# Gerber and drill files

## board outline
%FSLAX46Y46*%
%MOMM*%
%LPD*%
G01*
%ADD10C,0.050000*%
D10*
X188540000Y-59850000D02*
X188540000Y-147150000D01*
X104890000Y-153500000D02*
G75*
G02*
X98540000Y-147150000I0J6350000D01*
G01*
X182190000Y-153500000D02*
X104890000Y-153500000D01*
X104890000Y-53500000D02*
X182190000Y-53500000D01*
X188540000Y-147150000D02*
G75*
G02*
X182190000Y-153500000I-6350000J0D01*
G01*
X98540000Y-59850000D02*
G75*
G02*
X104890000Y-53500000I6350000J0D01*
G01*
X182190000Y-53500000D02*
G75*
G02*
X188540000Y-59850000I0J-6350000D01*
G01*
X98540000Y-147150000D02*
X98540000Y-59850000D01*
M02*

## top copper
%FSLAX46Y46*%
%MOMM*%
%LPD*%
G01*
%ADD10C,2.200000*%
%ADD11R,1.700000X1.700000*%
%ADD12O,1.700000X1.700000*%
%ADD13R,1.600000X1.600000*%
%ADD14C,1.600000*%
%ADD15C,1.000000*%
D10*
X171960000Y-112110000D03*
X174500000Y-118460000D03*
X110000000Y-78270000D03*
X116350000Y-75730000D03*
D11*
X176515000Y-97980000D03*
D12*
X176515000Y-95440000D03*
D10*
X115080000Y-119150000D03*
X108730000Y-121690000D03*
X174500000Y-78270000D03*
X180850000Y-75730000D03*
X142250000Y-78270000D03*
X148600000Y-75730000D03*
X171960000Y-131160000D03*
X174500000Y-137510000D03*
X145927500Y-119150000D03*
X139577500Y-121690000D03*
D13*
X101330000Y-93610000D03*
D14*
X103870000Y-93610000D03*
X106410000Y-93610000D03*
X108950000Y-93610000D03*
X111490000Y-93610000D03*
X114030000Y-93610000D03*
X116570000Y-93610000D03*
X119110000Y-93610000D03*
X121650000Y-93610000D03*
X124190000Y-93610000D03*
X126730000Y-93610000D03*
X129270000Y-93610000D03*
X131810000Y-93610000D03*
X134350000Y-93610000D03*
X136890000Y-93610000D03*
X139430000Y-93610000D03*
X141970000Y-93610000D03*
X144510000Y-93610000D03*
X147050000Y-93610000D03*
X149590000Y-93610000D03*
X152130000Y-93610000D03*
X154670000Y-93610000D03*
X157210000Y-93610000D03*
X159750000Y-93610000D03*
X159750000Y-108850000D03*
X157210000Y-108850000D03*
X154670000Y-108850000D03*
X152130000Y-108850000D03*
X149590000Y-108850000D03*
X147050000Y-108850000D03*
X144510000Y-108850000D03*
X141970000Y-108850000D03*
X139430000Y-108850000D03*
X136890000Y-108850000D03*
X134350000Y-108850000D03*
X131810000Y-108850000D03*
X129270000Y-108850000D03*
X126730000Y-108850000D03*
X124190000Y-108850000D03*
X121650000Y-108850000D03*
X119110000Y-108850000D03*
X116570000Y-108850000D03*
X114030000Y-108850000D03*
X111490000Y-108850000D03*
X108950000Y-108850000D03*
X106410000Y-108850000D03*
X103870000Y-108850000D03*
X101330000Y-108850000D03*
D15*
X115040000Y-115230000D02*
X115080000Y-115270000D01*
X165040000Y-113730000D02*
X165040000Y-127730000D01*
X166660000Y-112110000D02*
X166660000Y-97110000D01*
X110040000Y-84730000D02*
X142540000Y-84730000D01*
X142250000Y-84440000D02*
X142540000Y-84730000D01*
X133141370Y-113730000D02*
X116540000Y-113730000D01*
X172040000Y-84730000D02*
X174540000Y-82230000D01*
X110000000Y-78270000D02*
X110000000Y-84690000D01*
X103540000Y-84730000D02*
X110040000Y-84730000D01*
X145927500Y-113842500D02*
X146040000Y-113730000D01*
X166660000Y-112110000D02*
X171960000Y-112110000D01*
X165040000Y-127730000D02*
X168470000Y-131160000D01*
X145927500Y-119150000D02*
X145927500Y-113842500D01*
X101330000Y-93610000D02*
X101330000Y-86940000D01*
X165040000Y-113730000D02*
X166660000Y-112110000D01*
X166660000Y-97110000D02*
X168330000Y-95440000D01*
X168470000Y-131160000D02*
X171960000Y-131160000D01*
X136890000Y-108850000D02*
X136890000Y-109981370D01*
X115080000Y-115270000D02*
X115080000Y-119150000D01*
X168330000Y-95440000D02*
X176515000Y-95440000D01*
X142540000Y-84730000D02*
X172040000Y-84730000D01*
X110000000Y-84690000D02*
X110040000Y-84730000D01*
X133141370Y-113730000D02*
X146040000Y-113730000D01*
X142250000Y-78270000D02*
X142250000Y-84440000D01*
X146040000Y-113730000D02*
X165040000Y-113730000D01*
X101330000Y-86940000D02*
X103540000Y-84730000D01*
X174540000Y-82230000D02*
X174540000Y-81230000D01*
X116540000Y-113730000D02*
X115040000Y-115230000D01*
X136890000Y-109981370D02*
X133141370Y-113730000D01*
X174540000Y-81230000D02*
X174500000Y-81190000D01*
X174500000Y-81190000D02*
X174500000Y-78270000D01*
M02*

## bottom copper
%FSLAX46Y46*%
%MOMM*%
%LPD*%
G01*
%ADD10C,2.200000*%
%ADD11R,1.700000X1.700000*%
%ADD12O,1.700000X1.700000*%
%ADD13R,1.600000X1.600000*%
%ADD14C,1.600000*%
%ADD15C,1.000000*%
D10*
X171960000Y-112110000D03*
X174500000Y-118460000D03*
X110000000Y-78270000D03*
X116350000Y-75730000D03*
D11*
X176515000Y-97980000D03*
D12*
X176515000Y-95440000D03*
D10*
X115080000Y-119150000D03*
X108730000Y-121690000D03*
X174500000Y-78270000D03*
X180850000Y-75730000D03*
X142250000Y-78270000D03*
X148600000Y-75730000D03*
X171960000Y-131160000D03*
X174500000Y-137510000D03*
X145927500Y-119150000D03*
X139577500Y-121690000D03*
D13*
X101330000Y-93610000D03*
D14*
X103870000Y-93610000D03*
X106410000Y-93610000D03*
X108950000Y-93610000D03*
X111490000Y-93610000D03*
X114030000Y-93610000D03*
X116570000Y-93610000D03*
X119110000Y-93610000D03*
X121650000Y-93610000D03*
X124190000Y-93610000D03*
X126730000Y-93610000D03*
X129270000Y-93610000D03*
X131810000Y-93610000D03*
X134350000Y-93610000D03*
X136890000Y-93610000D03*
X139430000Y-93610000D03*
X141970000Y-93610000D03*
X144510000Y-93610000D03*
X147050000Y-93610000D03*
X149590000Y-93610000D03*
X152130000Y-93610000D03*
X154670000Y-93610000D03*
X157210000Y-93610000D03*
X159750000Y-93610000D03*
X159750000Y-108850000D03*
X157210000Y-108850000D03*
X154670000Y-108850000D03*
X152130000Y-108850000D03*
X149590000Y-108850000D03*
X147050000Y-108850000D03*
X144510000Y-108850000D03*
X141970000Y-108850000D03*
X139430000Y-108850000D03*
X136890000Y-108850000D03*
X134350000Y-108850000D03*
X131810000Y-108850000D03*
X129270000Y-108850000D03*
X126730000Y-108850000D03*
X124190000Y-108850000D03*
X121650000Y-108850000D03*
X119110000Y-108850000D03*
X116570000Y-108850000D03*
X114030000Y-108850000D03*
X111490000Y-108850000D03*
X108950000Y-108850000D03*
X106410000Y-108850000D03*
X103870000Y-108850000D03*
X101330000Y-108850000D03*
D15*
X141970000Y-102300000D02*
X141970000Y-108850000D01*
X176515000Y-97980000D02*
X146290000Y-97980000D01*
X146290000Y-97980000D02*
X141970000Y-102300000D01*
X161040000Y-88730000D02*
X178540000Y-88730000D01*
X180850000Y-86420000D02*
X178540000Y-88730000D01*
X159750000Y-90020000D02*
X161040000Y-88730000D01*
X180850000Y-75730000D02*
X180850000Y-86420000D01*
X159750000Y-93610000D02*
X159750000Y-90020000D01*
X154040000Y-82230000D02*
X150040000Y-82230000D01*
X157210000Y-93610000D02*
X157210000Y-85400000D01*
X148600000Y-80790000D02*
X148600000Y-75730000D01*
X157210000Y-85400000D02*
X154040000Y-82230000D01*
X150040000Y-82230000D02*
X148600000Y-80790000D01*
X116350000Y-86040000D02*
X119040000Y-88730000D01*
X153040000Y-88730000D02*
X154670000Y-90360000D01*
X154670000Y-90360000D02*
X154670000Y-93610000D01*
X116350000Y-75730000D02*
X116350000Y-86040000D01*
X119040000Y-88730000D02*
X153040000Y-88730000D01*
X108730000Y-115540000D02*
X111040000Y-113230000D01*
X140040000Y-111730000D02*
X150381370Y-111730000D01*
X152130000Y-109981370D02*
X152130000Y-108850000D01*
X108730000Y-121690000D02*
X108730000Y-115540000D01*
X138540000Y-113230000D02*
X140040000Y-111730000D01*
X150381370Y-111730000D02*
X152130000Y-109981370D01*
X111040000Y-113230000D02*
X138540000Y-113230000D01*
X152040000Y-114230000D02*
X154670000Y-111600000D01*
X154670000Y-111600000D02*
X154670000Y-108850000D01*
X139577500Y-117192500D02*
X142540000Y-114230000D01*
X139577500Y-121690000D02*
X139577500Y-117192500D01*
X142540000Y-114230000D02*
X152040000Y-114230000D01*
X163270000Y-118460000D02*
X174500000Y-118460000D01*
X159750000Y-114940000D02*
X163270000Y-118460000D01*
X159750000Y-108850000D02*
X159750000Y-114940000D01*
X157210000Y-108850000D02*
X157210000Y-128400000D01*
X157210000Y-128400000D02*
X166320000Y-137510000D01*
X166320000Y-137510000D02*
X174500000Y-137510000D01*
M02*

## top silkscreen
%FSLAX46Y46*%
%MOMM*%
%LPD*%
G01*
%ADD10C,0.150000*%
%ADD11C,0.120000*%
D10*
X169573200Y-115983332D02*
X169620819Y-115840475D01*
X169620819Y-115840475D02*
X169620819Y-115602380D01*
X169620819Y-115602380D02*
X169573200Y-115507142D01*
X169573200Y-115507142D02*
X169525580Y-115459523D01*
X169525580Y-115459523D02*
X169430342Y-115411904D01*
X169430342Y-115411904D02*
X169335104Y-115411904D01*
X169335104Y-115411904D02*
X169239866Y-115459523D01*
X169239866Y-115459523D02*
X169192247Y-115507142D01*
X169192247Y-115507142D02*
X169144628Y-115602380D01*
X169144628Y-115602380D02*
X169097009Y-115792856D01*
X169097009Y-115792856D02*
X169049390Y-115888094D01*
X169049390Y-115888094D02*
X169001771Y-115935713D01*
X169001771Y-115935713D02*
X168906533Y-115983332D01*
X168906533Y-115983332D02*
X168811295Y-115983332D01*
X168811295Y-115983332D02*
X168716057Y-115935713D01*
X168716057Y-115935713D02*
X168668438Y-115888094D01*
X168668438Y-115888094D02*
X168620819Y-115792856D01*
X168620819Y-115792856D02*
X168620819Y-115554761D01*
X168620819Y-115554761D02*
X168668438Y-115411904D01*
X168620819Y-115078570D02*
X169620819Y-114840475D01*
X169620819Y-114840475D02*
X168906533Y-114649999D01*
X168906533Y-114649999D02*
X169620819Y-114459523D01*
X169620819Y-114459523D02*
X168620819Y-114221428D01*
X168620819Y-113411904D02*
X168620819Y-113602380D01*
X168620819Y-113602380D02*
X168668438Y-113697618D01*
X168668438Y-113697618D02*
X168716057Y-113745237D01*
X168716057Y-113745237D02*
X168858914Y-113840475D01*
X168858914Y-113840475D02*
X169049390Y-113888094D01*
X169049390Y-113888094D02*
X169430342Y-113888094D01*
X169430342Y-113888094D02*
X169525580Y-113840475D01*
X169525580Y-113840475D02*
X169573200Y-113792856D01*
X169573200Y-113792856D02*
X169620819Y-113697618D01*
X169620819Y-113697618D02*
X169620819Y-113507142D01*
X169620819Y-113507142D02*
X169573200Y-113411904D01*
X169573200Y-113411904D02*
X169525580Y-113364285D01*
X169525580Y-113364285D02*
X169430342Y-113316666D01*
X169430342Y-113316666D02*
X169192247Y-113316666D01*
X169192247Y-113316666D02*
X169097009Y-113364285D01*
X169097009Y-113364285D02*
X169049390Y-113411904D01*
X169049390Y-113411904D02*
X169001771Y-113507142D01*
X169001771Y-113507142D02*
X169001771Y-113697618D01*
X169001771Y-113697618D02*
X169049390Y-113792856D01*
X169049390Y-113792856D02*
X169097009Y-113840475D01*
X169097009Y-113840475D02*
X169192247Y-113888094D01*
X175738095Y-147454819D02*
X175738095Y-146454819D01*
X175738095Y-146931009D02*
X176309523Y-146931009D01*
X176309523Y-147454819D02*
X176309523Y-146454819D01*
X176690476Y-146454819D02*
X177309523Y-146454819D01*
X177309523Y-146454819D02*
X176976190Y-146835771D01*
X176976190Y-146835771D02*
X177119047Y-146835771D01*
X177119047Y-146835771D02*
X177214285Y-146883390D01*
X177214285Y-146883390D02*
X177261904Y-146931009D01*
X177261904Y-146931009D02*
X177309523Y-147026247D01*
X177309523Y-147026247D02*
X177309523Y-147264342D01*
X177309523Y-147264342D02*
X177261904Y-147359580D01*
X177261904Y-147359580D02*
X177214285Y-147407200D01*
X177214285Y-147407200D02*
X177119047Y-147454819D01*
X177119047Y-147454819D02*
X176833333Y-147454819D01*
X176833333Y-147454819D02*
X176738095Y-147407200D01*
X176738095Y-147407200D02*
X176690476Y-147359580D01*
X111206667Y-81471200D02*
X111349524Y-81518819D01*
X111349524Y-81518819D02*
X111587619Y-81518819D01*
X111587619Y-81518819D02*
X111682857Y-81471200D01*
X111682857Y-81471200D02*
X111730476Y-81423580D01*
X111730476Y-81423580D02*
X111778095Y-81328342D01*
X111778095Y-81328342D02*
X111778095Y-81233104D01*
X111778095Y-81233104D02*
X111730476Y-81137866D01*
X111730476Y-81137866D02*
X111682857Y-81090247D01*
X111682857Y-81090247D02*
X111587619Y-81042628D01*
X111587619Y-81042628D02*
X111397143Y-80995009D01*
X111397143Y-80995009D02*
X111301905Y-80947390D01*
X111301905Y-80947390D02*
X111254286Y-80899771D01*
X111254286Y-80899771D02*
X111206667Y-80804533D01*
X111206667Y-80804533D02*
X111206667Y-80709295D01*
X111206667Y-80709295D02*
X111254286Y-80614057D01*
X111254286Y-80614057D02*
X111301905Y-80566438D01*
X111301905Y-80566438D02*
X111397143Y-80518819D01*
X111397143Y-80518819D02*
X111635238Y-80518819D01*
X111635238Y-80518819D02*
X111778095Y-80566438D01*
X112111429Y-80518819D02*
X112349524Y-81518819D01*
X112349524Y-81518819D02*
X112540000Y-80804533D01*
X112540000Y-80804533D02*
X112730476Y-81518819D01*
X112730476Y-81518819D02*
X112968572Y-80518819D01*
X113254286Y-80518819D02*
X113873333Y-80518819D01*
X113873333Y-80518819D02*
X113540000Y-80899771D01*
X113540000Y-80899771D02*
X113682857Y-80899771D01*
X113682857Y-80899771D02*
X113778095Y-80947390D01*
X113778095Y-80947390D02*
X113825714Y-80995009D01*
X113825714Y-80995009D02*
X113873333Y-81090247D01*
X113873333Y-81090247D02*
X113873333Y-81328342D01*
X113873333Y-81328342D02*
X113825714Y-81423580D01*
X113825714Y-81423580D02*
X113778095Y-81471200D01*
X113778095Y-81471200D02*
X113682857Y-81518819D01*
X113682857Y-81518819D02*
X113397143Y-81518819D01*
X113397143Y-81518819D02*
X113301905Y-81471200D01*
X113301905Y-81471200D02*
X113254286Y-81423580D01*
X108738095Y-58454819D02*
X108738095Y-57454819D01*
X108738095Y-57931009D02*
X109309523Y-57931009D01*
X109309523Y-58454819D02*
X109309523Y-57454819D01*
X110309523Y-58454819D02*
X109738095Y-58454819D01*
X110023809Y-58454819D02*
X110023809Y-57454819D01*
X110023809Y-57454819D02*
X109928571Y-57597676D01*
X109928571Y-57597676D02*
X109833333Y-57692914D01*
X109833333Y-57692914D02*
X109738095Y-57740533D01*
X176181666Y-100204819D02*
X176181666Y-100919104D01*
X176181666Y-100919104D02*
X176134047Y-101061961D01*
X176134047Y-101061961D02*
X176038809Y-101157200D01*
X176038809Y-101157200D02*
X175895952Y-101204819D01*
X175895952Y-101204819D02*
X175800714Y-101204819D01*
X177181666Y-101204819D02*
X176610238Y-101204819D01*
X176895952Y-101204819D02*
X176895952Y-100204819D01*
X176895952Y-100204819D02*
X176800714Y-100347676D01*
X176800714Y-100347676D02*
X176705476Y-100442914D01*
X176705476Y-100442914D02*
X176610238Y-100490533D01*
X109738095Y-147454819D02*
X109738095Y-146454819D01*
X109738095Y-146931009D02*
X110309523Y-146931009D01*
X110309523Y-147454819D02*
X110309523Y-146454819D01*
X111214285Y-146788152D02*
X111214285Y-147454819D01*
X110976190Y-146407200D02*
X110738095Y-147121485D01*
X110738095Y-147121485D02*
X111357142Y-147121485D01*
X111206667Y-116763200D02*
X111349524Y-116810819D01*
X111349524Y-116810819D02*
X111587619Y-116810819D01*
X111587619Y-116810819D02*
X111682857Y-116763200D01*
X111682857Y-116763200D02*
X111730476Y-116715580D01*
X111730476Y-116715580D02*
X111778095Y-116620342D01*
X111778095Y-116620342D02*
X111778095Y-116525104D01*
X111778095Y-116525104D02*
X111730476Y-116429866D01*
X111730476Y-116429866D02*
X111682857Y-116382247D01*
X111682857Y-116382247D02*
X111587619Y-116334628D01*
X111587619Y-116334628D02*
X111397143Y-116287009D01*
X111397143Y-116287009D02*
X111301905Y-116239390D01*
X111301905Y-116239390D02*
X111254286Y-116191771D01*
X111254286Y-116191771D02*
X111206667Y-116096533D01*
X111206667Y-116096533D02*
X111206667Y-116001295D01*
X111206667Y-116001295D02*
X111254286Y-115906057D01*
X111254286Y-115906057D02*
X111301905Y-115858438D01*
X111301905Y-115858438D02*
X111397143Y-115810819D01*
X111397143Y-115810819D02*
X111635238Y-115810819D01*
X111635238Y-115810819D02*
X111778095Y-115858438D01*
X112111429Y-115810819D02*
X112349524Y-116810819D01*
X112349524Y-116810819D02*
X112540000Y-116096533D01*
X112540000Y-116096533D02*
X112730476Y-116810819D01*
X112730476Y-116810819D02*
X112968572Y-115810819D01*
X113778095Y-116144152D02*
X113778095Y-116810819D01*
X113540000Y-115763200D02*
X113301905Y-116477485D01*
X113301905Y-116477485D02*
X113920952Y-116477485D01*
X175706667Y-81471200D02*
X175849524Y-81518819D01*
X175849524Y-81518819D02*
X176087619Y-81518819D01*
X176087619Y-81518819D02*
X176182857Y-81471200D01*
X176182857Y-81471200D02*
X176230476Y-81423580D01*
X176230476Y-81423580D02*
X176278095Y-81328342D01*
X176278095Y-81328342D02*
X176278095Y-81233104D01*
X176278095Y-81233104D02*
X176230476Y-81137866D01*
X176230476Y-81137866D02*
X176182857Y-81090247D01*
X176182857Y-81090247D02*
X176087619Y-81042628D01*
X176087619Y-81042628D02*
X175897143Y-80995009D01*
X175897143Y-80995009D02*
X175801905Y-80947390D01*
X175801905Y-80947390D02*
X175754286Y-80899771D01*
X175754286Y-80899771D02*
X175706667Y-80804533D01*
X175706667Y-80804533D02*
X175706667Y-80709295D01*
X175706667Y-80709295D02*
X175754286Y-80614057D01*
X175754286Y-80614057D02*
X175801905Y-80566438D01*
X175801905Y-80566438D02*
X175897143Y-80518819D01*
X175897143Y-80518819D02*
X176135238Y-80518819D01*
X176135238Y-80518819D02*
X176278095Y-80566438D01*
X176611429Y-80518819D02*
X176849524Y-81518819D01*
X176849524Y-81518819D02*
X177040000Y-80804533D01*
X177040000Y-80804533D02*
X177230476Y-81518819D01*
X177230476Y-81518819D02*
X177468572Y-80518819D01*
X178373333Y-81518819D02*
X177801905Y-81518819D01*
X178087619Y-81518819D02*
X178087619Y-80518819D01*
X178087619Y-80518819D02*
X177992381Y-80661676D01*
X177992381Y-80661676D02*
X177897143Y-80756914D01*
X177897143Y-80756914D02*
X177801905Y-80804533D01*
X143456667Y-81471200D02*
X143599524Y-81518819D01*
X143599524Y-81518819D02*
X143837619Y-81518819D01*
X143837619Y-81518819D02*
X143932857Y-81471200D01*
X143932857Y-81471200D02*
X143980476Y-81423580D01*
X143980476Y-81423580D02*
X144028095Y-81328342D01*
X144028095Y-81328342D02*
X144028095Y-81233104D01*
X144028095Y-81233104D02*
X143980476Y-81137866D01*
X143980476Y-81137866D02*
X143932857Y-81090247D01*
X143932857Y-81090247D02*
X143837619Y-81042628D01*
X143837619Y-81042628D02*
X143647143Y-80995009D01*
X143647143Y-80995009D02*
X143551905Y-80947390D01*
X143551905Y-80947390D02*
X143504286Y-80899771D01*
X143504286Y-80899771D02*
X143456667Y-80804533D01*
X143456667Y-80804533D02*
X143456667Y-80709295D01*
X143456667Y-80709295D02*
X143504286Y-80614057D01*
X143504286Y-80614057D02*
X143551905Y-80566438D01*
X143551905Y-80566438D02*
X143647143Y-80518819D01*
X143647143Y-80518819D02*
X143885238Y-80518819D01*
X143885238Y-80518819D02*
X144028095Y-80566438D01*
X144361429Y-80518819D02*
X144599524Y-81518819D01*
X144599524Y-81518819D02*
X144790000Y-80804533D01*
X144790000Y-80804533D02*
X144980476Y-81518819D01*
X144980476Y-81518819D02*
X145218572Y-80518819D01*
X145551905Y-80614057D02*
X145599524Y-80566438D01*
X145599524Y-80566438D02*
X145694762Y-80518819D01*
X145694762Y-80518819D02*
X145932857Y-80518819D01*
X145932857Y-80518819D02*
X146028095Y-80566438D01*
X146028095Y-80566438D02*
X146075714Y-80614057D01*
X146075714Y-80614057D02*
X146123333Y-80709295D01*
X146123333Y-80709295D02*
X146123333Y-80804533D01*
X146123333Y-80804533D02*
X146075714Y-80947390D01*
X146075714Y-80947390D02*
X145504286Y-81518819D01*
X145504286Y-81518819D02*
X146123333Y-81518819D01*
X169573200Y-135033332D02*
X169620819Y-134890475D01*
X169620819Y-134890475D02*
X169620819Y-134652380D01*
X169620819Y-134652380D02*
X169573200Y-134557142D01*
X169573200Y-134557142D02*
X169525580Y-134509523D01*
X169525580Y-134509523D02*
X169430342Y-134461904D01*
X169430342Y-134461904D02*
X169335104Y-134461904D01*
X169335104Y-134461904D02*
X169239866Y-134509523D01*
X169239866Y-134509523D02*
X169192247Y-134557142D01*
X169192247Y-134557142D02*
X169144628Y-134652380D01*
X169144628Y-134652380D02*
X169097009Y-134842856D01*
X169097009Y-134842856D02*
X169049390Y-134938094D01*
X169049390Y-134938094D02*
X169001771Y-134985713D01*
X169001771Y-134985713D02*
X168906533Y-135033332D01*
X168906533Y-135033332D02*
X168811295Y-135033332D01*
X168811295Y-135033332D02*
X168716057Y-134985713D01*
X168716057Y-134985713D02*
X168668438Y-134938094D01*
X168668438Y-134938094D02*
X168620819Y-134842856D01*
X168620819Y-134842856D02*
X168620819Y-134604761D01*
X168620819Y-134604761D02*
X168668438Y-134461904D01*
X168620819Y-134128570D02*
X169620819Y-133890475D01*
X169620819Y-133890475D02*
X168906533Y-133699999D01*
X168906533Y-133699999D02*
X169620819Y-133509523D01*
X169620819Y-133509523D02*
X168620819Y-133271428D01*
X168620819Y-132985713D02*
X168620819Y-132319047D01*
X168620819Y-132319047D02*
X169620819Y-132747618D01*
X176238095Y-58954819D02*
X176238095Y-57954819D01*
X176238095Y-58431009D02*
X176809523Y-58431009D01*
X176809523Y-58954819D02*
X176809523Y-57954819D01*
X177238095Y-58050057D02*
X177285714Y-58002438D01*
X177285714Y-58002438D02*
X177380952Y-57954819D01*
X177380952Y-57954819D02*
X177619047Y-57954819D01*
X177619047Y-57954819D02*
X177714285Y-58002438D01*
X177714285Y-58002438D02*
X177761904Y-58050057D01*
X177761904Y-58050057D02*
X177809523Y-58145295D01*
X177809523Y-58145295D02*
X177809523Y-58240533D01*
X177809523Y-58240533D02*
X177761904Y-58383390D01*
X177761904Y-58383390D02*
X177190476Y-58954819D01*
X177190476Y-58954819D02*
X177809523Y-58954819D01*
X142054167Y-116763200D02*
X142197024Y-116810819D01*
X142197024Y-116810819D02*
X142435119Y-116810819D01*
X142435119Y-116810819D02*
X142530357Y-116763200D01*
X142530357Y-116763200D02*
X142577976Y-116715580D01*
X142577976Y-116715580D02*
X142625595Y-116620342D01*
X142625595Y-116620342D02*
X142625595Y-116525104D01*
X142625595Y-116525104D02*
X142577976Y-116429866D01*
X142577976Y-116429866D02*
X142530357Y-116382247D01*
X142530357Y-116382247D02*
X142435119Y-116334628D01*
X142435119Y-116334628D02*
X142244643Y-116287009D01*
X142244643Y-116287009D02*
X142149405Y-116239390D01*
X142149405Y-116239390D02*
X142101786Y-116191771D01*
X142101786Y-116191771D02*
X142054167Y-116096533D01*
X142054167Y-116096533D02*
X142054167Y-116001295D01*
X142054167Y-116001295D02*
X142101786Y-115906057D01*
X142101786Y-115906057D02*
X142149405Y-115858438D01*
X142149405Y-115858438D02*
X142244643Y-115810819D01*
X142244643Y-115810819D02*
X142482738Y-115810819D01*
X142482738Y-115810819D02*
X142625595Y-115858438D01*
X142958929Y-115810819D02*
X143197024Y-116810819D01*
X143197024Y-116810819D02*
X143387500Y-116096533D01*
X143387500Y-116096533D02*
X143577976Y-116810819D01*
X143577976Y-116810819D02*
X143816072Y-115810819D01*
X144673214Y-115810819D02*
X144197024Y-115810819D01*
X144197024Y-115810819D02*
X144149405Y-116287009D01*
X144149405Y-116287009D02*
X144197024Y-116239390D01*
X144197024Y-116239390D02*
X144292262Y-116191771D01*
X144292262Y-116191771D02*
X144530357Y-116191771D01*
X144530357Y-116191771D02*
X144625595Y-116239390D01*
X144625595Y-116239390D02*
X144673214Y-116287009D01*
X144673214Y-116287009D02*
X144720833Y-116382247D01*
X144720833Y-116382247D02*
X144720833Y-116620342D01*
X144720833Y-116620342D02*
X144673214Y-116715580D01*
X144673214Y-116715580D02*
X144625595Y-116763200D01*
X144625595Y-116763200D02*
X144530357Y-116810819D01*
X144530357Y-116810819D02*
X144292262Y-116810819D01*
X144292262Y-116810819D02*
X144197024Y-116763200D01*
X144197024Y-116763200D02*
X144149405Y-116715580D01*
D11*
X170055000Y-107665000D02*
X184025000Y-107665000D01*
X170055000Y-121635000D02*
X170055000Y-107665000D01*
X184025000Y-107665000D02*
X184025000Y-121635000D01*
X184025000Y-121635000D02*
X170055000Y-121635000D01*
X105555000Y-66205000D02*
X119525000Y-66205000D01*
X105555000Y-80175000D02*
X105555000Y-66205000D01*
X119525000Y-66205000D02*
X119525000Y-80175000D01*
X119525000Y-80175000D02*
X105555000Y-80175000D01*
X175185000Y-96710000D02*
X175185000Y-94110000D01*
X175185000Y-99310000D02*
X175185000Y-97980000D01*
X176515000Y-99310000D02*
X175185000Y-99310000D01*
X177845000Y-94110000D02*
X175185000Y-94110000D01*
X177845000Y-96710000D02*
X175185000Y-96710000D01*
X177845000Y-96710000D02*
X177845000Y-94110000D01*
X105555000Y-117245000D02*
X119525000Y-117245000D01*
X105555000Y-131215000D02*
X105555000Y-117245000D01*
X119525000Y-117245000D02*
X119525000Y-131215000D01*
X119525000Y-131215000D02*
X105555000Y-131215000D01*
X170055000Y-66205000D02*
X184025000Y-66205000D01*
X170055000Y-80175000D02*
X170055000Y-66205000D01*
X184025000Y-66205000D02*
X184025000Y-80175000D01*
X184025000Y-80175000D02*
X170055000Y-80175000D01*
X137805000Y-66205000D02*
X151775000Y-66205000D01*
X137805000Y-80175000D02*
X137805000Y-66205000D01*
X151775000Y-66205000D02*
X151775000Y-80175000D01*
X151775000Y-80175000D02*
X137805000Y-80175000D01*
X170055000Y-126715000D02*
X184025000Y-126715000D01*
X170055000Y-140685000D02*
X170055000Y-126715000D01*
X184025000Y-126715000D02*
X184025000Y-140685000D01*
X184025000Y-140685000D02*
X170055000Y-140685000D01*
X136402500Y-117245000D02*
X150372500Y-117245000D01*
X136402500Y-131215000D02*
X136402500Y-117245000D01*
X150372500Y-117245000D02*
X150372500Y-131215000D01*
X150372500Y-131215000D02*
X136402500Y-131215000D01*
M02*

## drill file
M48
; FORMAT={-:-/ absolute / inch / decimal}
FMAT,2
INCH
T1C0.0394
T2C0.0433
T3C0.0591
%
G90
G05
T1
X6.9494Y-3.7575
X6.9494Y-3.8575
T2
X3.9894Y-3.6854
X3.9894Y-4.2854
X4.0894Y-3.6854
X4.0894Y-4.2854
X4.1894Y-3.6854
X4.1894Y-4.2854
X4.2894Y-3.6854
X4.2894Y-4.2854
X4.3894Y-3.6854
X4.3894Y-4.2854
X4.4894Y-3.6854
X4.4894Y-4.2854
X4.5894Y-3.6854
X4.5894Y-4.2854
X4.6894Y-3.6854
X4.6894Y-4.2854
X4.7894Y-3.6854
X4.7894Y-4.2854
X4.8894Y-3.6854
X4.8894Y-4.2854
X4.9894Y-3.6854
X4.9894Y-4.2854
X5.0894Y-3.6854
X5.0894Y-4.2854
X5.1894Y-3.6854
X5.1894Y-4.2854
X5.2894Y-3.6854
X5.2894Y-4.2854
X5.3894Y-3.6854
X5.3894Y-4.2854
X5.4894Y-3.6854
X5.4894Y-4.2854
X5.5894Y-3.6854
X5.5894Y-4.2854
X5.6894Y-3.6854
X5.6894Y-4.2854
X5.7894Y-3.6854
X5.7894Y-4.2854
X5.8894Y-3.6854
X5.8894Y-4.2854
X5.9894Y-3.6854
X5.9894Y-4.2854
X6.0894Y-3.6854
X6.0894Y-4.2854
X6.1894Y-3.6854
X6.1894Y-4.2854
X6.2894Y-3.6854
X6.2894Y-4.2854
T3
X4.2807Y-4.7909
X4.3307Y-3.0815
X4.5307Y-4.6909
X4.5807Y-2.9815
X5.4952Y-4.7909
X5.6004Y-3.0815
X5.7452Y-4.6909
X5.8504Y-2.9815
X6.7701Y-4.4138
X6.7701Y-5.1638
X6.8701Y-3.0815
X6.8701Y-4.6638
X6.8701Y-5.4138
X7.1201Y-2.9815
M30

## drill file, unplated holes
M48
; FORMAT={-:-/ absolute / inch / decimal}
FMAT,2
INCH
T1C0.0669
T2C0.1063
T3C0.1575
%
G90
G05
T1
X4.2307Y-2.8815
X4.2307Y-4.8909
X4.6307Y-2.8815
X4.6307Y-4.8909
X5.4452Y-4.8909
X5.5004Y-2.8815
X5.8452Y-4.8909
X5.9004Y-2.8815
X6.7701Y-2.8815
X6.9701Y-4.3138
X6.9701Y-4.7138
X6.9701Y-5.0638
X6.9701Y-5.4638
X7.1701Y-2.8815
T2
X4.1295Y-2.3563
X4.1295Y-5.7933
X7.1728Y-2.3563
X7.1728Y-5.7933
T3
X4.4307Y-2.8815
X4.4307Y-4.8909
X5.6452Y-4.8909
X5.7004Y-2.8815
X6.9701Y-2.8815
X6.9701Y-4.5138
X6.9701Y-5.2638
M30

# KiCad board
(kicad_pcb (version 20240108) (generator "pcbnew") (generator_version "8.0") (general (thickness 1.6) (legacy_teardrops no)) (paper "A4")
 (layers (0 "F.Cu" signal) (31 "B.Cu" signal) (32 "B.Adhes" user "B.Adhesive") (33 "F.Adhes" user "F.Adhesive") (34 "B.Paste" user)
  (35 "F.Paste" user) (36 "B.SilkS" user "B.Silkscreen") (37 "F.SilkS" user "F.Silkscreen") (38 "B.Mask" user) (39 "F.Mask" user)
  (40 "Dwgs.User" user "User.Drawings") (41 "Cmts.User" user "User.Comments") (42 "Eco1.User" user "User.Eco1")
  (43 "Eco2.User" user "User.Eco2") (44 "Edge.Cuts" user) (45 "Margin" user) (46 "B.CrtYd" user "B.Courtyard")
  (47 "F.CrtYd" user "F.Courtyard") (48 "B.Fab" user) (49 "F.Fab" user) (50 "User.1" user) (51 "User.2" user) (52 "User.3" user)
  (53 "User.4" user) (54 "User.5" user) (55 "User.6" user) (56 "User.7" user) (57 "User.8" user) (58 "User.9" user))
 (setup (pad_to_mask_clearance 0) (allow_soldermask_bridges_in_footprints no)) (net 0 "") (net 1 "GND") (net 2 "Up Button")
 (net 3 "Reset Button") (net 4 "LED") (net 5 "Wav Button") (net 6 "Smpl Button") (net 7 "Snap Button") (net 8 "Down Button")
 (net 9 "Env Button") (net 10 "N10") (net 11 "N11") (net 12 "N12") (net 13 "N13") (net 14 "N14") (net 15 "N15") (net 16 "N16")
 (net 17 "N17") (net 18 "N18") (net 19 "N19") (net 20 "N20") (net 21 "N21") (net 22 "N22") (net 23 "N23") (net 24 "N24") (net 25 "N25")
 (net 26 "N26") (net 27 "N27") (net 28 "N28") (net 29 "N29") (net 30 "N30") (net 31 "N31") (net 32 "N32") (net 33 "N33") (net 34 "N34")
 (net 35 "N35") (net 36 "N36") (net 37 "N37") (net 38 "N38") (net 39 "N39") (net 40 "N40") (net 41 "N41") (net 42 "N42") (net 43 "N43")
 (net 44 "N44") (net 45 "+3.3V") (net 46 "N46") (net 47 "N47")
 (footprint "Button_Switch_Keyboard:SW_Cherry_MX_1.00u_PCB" (layer "F.Cu") (at 171.96 112.11 90)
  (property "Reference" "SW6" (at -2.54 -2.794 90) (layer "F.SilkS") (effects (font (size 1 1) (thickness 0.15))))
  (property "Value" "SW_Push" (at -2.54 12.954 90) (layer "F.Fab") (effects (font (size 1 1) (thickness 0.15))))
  (fp_line (start 4.445 -1.905) (end 4.445 12.065) (stroke (width 0.12) (type solid)) (layer "F.SilkS"))
  (fp_line (start -9.525 -1.905) (end 4.445 -1.905) (stroke (width 0.12) (type solid)) (layer "F.SilkS"))
  (fp_line (start 4.445 12.065) (end -9.525 12.065) (stroke (width 0.12) (type solid)) (layer "F.SilkS"))
  (fp_line (start -9.525 12.065) (end -9.525 -1.905) (stroke (width 0.12) (type solid)) (layer "F.SilkS"))
  (pad "" np_thru_hole circle (at -7.62 5.08 90) (size 1.7 1.7) (drill 1.7) (layers "*.Cu" "*.Mask"))
  (pad "" np_thru_hole circle (at -2.54 5.08 90) (size 4 4) (drill 4) (layers "*.Cu" "*.Mask"))
  (pad "" np_thru_hole circle (at 2.54 5.08 90) (size 1.7 1.7) (drill 1.7) (layers "*.Cu" "*.Mask"))
  (pad "1" thru_hole circle (at 0 0 90) (size 2.2 2.2) (drill 1.5) (layers "*.Cu" "*.Mask") (remove_unused_layers no) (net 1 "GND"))
  (pad "2" thru_hole circle (at -6.35 2.54 90) (size 2.2 2.2) (drill 1.5) (layers "*.Cu" "*.Mask") (remove_unused_layers no)
   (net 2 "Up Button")))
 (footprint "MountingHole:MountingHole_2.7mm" (layer "F.Cu") (at 182.19 147.15)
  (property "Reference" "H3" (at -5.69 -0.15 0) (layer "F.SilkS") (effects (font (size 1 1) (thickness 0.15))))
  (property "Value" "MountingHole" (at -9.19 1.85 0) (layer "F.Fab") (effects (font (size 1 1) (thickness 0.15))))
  (pad "" np_thru_hole circle (at 0 0) (size 2.7 2.7) (drill 2.7) (layers "*.Cu" "*.Mask")))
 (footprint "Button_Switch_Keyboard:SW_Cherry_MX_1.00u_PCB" (layer "F.Cu") (at 110 78.27 180)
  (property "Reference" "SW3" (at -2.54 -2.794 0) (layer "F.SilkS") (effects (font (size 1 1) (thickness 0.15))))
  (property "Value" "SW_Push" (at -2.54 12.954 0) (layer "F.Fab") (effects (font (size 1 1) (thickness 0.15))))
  (fp_line (start 4.445 12.065) (end -9.525 12.065) (stroke (width 0.12) (type solid)) (layer "F.SilkS"))
  (fp_line (start 4.445 -1.905) (end 4.445 12.065) (stroke (width 0.12) (type solid)) (layer "F.SilkS"))
  (fp_line (start -9.525 12.065) (end -9.525 -1.905) (stroke (width 0.12) (type solid)) (layer "F.SilkS"))
  (fp_line (start -9.525 -1.905) (end 4.445 -1.905) (stroke (width 0.12) (type solid)) (layer "F.SilkS"))
  (pad "" np_thru_hole circle (at -7.62 5.08 180) (size 1.7 1.7) (drill 1.7) (layers "*.Cu" "*.Mask"))
  (pad "" np_thru_hole circle (at -2.54 5.08 180) (size 4 4) (drill 4) (layers "*.Cu" "*.Mask"))
  (pad "" np_thru_hole circle (at 2.54 5.08 180) (size 1.7 1.7) (drill 1.7) (layers "*.Cu" "*.Mask"))
  (pad "1" thru_hole circle (at 0 0 180) (size 2.2 2.2) (drill 1.5) (layers "*.Cu" "*.Mask") (remove_unused_layers no) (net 1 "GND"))
  (pad "2" thru_hole circle (at -6.35 2.54 180) (size 2.2 2.2) (drill 1.5) (layers "*.Cu" "*.Mask") (remove_unused_layers no)
   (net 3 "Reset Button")))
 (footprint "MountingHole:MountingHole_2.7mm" (layer "F.Cu") (at 104.89 59.85)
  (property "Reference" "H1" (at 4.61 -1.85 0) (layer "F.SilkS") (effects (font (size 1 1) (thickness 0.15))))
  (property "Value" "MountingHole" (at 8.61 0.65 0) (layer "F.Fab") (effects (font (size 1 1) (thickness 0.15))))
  (pad "" np_thru_hole circle (at 0 0) (size 2.7 2.7) (drill 2.7) (layers "*.Cu" "*.Mask")))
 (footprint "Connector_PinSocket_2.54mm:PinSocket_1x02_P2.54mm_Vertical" (layer "F.Cu") (at 176.515 97.98 180)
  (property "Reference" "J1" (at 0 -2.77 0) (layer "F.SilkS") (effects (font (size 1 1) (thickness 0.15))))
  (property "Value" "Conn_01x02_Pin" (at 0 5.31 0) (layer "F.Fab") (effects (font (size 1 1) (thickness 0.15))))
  (fp_line (start 1.33 1.27) (end 1.33 3.87) (stroke (width 0.12) (type solid)) (layer "F.SilkS"))
  (fp_line (start 1.33 -1.33) (end 1.33 0) (stroke (width 0.12) (type solid)) (layer "F.SilkS"))
  (fp_line (start 0 -1.33) (end 1.33 -1.33) (stroke (width 0.12) (type solid)) (layer "F.SilkS"))
  (fp_line (start -1.33 3.87) (end 1.33 3.87) (stroke (width 0.12) (type solid)) (layer "F.SilkS"))
  (fp_line (start -1.33 1.27) (end 1.33 1.27) (stroke (width 0.12) (type solid)) (layer "F.SilkS"))
  (fp_line (start -1.33 1.27) (end -1.33 3.87) (stroke (width 0.12) (type solid)) (layer "F.SilkS"))
  (pad "1" thru_hole rect (at 0 0 180) (size 1.7 1.7) (drill 1) (layers "*.Cu" "*.Mask") (remove_unused_layers no) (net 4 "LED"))
  (pad "2" thru_hole oval (at 0 2.54 180) (size 1.7 1.7) (drill 1) (layers "*.Cu" "*.Mask") (remove_unused_layers no) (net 1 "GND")))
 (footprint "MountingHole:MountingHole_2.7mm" (layer "F.Cu") (at 104.89 147.15)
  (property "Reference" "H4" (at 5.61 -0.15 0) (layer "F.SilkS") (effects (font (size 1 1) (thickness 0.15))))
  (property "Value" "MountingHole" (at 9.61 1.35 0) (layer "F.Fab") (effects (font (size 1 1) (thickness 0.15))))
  (pad "" np_thru_hole circle (at 0 0) (size 2.7 2.7) (drill 2.7) (layers "*.Cu" "*.Mask")))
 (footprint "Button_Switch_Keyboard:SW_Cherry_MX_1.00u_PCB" (layer "F.Cu") (at 115.08 119.15)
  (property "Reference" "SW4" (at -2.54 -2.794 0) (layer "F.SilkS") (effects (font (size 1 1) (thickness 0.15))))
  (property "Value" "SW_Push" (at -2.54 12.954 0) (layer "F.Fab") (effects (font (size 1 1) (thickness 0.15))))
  (fp_line (start -9.525 -1.905) (end 4.445 -1.905) (stroke (width 0.12) (type solid)) (layer "F.SilkS"))
  (fp_line (start -9.525 12.065) (end -9.525 -1.905) (stroke (width 0.12) (type solid)) (layer "F.SilkS"))
  (fp_line (start 4.445 -1.905) (end 4.445 12.065) (stroke (width 0.12) (type solid)) (layer "F.SilkS"))
  (fp_line (start 4.445 12.065) (end -9.525 12.065) (stroke (width 0.12) (type solid)) (layer "F.SilkS"))
  (pad "" np_thru_hole circle (at -7.62 5.08) (size 1.7 1.7) (drill 1.7) (layers "*.Cu" "*.Mask"))
  (pad "" np_thru_hole circle (at -2.54 5.08) (size 4 4) (drill 4) (layers "*.Cu" "*.Mask"))
  (pad "" np_thru_hole circle (at 2.54 5.08) (size 1.7 1.7) (drill 1.7) (layers "*.Cu" "*.Mask"))
  (pad "1" thru_hole circle (at 0 0) (size 2.2 2.2) (drill 1.5) (layers "*.Cu" "*.Mask") (remove_unused_layers no) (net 1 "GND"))
  (pad "2" thru_hole circle (at -6.35 2.54) (size 2.2 2.2) (drill 1.5) (layers "*.Cu" "*.Mask") (remove_unused_layers no)
   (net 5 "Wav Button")))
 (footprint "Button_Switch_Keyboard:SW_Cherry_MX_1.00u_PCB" (layer "F.Cu") (at 174.5 78.27 180)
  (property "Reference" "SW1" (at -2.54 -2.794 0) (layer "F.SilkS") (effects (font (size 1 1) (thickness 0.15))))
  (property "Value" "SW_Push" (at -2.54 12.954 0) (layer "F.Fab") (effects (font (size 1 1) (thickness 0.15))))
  (fp_line (start 4.445 12.065) (end -9.525 12.065) (stroke (width 0.12) (type solid)) (layer "F.SilkS"))
  (fp_line (start 4.445 -1.905) (end 4.445 12.065) (stroke (width 0.12) (type solid)) (layer "F.SilkS"))
  (fp_line (start -9.525 12.065) (end -9.525 -1.905) (stroke (width 0.12) (type solid)) (layer "F.SilkS"))
  (fp_line (start -9.525 -1.905) (end 4.445 -1.905) (stroke (width 0.12) (type solid)) (layer "F.SilkS"))
  (pad "" np_thru_hole circle (at -7.62 5.08 180) (size 1.7 1.7) (drill 1.7) (layers "*.Cu" "*.Mask"))
  (pad "" np_thru_hole circle (at -2.54 5.08 180) (size 4 4) (drill 4) (layers "*.Cu" "*.Mask"))
  (pad "" np_thru_hole circle (at 2.54 5.08 180) (size 1.7 1.7) (drill 1.7) (layers "*.Cu" "*.Mask"))
  (pad "1" thru_hole circle (at 0 0 180) (size 2.2 2.2) (drill 1.5) (layers "*.Cu" "*.Mask") (remove_unused_layers no) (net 1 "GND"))
  (pad "2" thru_hole circle (at -6.35 2.54 180) (size 2.2 2.2) (drill 1.5) (layers "*.Cu" "*.Mask") (remove_unused_layers no)
   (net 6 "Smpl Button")))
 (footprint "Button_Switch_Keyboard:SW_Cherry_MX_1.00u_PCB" (layer "F.Cu") (at 142.25 78.27 180)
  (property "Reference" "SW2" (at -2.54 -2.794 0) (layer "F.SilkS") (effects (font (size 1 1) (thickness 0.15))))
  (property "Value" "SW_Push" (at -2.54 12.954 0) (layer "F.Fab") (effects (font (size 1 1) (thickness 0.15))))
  (fp_line (start 4.445 12.065) (end -9.525 12.065) (stroke (width 0.12) (type solid)) (layer "F.SilkS"))
  (fp_line (start 4.445 -1.905) (end 4.445 12.065) (stroke (width 0.12) (type solid)) (layer "F.SilkS"))
  (fp_line (start -9.525 12.065) (end -9.525 -1.905) (stroke (width 0.12) (type solid)) (layer "F.SilkS"))
  (fp_line (start -9.525 -1.905) (end 4.445 -1.905) (stroke (width 0.12) (type solid)) (layer "F.SilkS"))
  (pad "" np_thru_hole circle (at -7.62 5.08 180) (size 1.7 1.7) (drill 1.7) (layers "*.Cu" "*.Mask"))
  (pad "" np_thru_hole circle (at -2.54 5.08 180) (size 4 4) (drill 4) (layers "*.Cu" "*.Mask"))
  (pad "" np_thru_hole circle (at 2.54 5.08 180) (size 1.7 1.7) (drill 1.7) (layers "*.Cu" "*.Mask"))
  (pad "1" thru_hole circle (at 0 0 180) (size 2.2 2.2) (drill 1.5) (layers "*.Cu" "*.Mask") (remove_unused_layers no) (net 1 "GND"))
  (pad "2" thru_hole circle (at -6.35 2.54 180) (size 2.2 2.2) (drill 1.5) (layers "*.Cu" "*.Mask") (remove_unused_layers no)
   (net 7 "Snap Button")))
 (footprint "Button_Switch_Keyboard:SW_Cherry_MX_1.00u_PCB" (layer "F.Cu") (at 171.96 131.16 90)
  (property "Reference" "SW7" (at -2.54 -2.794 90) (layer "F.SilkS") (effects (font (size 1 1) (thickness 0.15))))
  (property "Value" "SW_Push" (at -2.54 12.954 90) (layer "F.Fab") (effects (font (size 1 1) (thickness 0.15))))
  (fp_line (start 4.445 -1.905) (end 4.445 12.065) (stroke (width 0.12) (type solid)) (layer "F.SilkS"))
  (fp_line (start -9.525 -1.905) (end 4.445 -1.905) (stroke (width 0.12) (type solid)) (layer "F.SilkS"))
  (fp_line (start 4.445 12.065) (end -9.525 12.065) (stroke (width 0.12) (type solid)) (layer "F.SilkS"))
  (fp_line (start -9.525 12.065) (end -9.525 -1.905) (stroke (width 0.12) (type solid)) (layer "F.SilkS"))
  (pad "" np_thru_hole circle (at -7.62 5.08 90) (size 1.7 1.7) (drill 1.7) (layers "*.Cu" "*.Mask"))
  (pad "" np_thru_hole circle (at -2.54 5.08 90) (size 4 4) (drill 4) (layers "*.Cu" "*.Mask"))
  (pad "" np_thru_hole circle (at 2.54 5.08 90) (size 1.7 1.7) (drill 1.7) (layers "*.Cu" "*.Mask"))
  (pad "1" thru_hole circle (at 0 0 90) (size 2.2 2.2) (drill 1.5) (layers "*.Cu" "*.Mask") (remove_unused_layers no) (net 1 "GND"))
  (pad "2" thru_hole circle (at -6.35 2.54 90) (size 2.2 2.2) (drill 1.5) (layers "*.Cu" "*.Mask") (remove_unused_layers no)
   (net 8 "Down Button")))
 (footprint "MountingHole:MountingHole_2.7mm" (layer "F.Cu") (at 182.19 59.85)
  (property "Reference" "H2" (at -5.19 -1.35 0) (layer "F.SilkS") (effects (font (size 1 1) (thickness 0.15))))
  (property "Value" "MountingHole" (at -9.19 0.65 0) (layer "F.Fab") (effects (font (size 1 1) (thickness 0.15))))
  (pad "" np_thru_hole circle (at 0 0) (size 2.7 2.7) (drill 2.7) (layers "*.Cu" "*.Mask")))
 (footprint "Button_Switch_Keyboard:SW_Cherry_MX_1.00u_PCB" (layer "F.Cu") (at 145.9275 119.15)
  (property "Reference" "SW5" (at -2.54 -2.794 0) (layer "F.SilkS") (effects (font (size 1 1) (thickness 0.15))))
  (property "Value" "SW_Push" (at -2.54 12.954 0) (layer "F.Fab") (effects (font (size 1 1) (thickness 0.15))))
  (fp_line (start -9.525 -1.905) (end 4.445 -1.905) (stroke (width 0.12) (type solid)) (layer "F.SilkS"))
  (fp_line (start -9.525 12.065) (end -9.525 -1.905) (stroke (width 0.12) (type solid)) (layer "F.SilkS"))
  (fp_line (start 4.445 -1.905) (end 4.445 12.065) (stroke (width 0.12) (type solid)) (layer "F.SilkS"))
  (fp_line (start 4.445 12.065) (end -9.525 12.065) (stroke (width 0.12) (type solid)) (layer "F.SilkS"))
  (pad "" np_thru_hole circle (at -7.62 5.08) (size 1.7 1.7) (drill 1.7) (layers "*.Cu" "*.Mask"))
  (pad "" np_thru_hole circle (at -2.54 5.08) (size 4 4) (drill 4) (layers "*.Cu" "*.Mask"))
  (pad "" np_thru_hole circle (at 2.54 5.08) (size 1.7 1.7) (drill 1.7) (layers "*.Cu" "*.Mask"))
  (pad "1" thru_hole circle (at 0 0) (size 2.2 2.2) (drill 1.5) (layers "*.Cu" "*.Mask") (remove_unused_layers no) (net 1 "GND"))
  (pad "2" thru_hole circle (at -6.35 2.54) (size 2.2 2.2) (drill 1.5) (layers "*.Cu" "*.Mask") (remove_unused_layers no)
   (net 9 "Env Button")))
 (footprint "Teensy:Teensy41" (layer "B.Cu") (at 130.54 101.23)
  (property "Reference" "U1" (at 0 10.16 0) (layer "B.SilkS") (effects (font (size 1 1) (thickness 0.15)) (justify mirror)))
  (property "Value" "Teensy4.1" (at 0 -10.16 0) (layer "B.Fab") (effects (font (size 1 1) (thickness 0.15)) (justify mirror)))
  (pad "1" thru_hole rect (at -29.21 -7.62) (size 1.6 1.6) (drill 1.1) (layers "*.Cu" "*.Mask") (remove_unused_layers no) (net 1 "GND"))
  (pad "2" thru_hole circle (at -26.67 -7.62) (size 1.6 1.6) (drill 1.1) (layers "*.Cu" "*.Mask") (remove_unused_layers no) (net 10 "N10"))
  (pad "3" thru_hole circle (at -24.13 -7.62) (size 1.6 1.6) (drill 1.1) (layers "*.Cu" "*.Mask") (remove_unused_layers no) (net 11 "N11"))
  (pad "4" thru_hole circle (at -21.59 -7.62) (size 1.6 1.6) (drill 1.1) (layers "*.Cu" "*.Mask") (remove_unused_layers no) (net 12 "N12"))
  (pad "5" thru_hole circle (at -19.05 -7.62) (size 1.6 1.6) (drill 1.1) (layers "*.Cu" "*.Mask") (remove_unused_layers no) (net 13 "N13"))
  (pad "6" thru_hole circle (at -16.51 -7.62) (size 1.6 1.6) (drill 1.1) (layers "*.Cu" "*.Mask") (remove_unused_layers no) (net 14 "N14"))
  (pad "7" thru_hole circle (at -13.97 -7.62) (size 1.6 1.6) (drill 1.1) (layers "*.Cu" "*.Mask") (remove_unused_layers no) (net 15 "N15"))
  (pad "8" thru_hole circle (at -11.43 -7.62) (size 1.6 1.6) (drill 1.1) (layers "*.Cu" "*.Mask") (remove_unused_layers no) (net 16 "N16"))
  (pad "9" thru_hole circle (at -8.89 -7.62) (size 1.6 1.6) (drill 1.1) (layers "*.Cu" "*.Mask") (remove_unused_layers no) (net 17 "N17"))
  (pad "10" thru_hole circle (at -6.35 -7.62) (size 1.6 1.6) (drill 1.1) (layers "*.Cu" "*.Mask") (remove_unused_layers no) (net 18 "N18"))
  (pad "11" thru_hole circle (at -3.81 -7.62) (size 1.6 1.6) (drill 1.1) (layers "*.Cu" "*.Mask") (remove_unused_layers no) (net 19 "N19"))
  (pad "12" thru_hole circle (at -1.27 -7.62) (size 1.6 1.6) (drill 1.1) (layers "*.Cu" "*.Mask") (remove_unused_layers no) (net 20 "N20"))
  (pad "13" thru_hole circle (at 1.27 -7.62) (size 1.6 1.6) (drill 1.1) (layers "*.Cu" "*.Mask") (remove_unused_layers no) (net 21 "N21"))
  (pad "14" thru_hole circle (at 3.81 -7.62) (size 1.6 1.6) (drill 1.1) (layers "*.Cu" "*.Mask") (remove_unused_layers no) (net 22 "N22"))
  (pad "15" thru_hole circle (at 6.35 -7.62) (size 1.6 1.6) (drill 1.1) (layers "*.Cu" "*.Mask") (remove_unused_layers no) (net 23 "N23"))
  (pad "16" thru_hole circle (at 8.89 -7.62) (size 1.6 1.6) (drill 1.1) (layers "*.Cu" "*.Mask") (remove_unused_layers no) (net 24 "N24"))
  (pad "17" thru_hole circle (at 11.43 -7.62) (size 1.6 1.6) (drill 1.1) (layers "*.Cu" "*.Mask") (remove_unused_layers no) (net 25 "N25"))
  (pad "18" thru_hole circle (at 13.97 -7.62) (size 1.6 1.6) (drill 1.1) (layers "*.Cu" "*.Mask") (remove_unused_layers no) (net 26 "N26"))
  (pad "19" thru_hole circle (at 16.51 -7.62) (size 1.6 1.6) (drill 1.1) (layers "*.Cu" "*.Mask") (remove_unused_layers no) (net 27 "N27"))
  (pad "20" thru_hole circle (at 19.05 -7.62) (size 1.6 1.6) (drill 1.1) (layers "*.Cu" "*.Mask") (remove_unused_layers no) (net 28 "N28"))
  (pad "21" thru_hole circle (at 21.59 -7.62) (size 1.6 1.6) (drill 1.1) (layers "*.Cu" "*.Mask") (remove_unused_layers no) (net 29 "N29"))
  (pad "22" thru_hole circle (at 24.13 -7.62) (size 1.6 1.6) (drill 1.1) (layers "*.Cu" "*.Mask") (remove_unused_layers no)
   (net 3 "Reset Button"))
  (pad "23" thru_hole circle (at 26.67 -7.62) (size 1.6 1.6) (drill 1.1) (layers "*.Cu" "*.Mask") (remove_unused_layers no)
   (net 7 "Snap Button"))
  (pad "24" thru_hole circle (at 29.21 -7.62) (size 1.6 1.6) (drill 1.1) (layers "*.Cu" "*.Mask") (remove_unused_layers no)
   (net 6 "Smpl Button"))
  (pad "25" thru_hole circle (at 29.21 7.62) (size 1.6 1.6) (drill 1.1) (layers "*.Cu" "*.Mask") (remove_unused_layers no)
   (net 2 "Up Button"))
  (pad "26" thru_hole circle (at 26.67 7.62) (size 1.6 1.6) (drill 1.1) (layers "*.Cu" "*.Mask") (remove_unused_layers no)
   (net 8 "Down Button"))
  (pad "27" thru_hole circle (at 24.13 7.62) (size 1.6 1.6) (drill 1.1) (layers "*.Cu" "*.Mask") (remove_unused_layers no)
   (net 9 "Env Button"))
  (pad "28" thru_hole circle (at 21.59 7.62) (size 1.6 1.6) (drill 1.1) (layers "*.Cu" "*.Mask") (remove_unused_layers no)
   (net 5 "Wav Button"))
  (pad "29" thru_hole circle (at 19.05 7.62) (size 1.6 1.6) (drill 1.1) (layers "*.Cu" "*.Mask") (remove_unused_layers no) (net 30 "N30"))
  (pad "30" thru_hole circle (at 16.51 7.62) (size 1.6 1.6) (drill 1.1) (layers "*.Cu" "*.Mask") (remove_unused_layers no) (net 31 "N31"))
  (pad "31" thru_hole circle (at 13.97 7.62) (size 1.6 1.6) (drill 1.1) (layers "*.Cu" "*.Mask") (remove_unused_layers no) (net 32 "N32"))
  (pad "32" thru_hole circle (at 11.43 7.62) (size 1.6 1.6) (drill 1.1) (layers "*.Cu" "*.Mask") (remove_unused_layers no) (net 4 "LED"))
  (pad "33" thru_hole circle (at 8.89 7.62) (size 1.6 1.6) (drill 1.1) (layers "*.Cu" "*.Mask") (remove_unused_layers no) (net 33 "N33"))
  (pad "34" thru_hole circle (at 6.35 7.62) (size 1.6 1.6) (drill 1.1) (layers "*.Cu" "*.Mask") (remove_unused_layers no) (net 1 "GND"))
  (pad "35" thru_hole circle (at 3.81 7.62) (size 1.6 1.6) (drill 1.1) (layers "*.Cu" "*.Mask") (remove_unused_layers no) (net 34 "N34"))
  (pad "36" thru_hole circle (at 1.27 7.62) (size 1.6 1.6) (drill 1.1) (layers "*.Cu" "*.Mask") (remove_unused_layers no) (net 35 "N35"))
  (pad "37" thru_hole circle (at -1.27 7.62) (size 1.6 1.6) (drill 1.1) (layers "*.Cu" "*.Mask") (remove_unused_layers no) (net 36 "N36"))
  (pad "38" thru_hole circle (at -3.81 7.62) (size 1.6 1.6) (drill 1.1) (layers "*.Cu" "*.Mask") (remove_unused_layers no) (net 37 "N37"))
  (pad "39" thru_hole circle (at -6.35 7.62) (size 1.6 1.6) (drill 1.1) (layers "*.Cu" "*.Mask") (remove_unused_layers no) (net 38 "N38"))
  (pad "40" thru_hole circle (at -8.89 7.62) (size 1.6 1.6) (drill 1.1) (layers "*.Cu" "*.Mask") (remove_unused_layers no) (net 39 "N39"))
  (pad "41" thru_hole circle (at -11.43 7.62) (size 1.6 1.6) (drill 1.1) (layers "*.Cu" "*.Mask") (remove_unused_layers no) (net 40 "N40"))
  (pad "42" thru_hole circle (at -13.97 7.62) (size 1.6 1.6) (drill 1.1) (layers "*.Cu" "*.Mask") (remove_unused_layers no) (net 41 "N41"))
  (pad "43" thru_hole circle (at -16.51 7.62) (size 1.6 1.6) (drill 1.1) (layers "*.Cu" "*.Mask") (remove_unused_layers no) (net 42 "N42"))
  (pad "44" thru_hole circle (at -19.05 7.62) (size 1.6 1.6) (drill 1.1) (layers "*.Cu" "*.Mask") (remove_unused_layers no) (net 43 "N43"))
  (pad "45" thru_hole circle (at -21.59 7.62) (size 1.6 1.6) (drill 1.1) (layers "*.Cu" "*.Mask") (remove_unused_layers no) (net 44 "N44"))
  (pad "46" thru_hole circle (at -24.13 7.62) (size 1.6 1.6) (drill 1.1) (layers "*.Cu" "*.Mask") (remove_unused_layers no) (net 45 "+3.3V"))
  (pad "47" thru_hole circle (at -26.67 7.62) (size 1.6 1.6) (drill 1.1) (layers "*.Cu" "*.Mask") (remove_unused_layers no) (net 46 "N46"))
  (pad "48" thru_hole circle (at -29.21 7.62) (size 1.6 1.6) (drill 1.1) (layers "*.Cu" "*.Mask") (remove_unused_layers no) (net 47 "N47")))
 (gr_line (start 188.54 59.85) (end 188.54 147.15) (stroke (width 0.05) (type default)) (layer "Edge.Cuts"))
 (gr_arc (start 104.89 153.5) (mid 100.399872 151.640128) (end 98.54 147.15) (stroke (width 0.05) (type default)) (layer "Edge.Cuts"))
 (gr_line (start 182.19 153.5) (end 104.89 153.5) (stroke (width 0.05) (type default)) (layer "Edge.Cuts"))
 (gr_line (start 104.89 53.5) (end 182.19 53.5) (stroke (width 0.05) (type default)) (layer "Edge.Cuts"))
 (gr_arc (start 188.54 147.15) (mid 186.680128 151.640128) (end 182.19 153.5) (stroke (width 0.05) (type default)) (layer "Edge.Cuts"))
 (gr_arc (start 98.54 59.85) (mid 100.399872 55.359872) (end 104.89 53.5) (stroke (width 0.05) (type default)) (layer "Edge.Cuts"))
 (gr_arc (start 182.19 53.5) (mid 186.680128 55.359872) (end 188.54 59.85) (stroke (width 0.05) (type default)) (layer "Edge.Cuts"))
 (gr_line (start 98.54 147.15) (end 98.54 59.85) (stroke (width 0.05) (type default)) (layer "Edge.Cuts"))
 (segment (start 141.97 102.3) (end 141.97 108.85) (width 1) (layer "B.Cu") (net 4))
 (segment (start 176.515 97.98) (end 146.29 97.98) (width 1) (layer "B.Cu") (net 4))
 (segment (start 146.29 97.98) (end 141.97 102.3) (width 1) (layer "B.Cu") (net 4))
 (segment (start 115.04 115.23) (end 115.08 115.27) (width 1) (layer "F.Cu") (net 1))
 (segment (start 165.04 113.73) (end 165.04 127.73) (width 1) (layer "F.Cu") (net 1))
 (segment (start 166.66 112.11) (end 166.66 97.11) (width 1) (layer "F.Cu") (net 1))
 (segment (start 110.04 84.73) (end 142.54 84.73) (width 1) (layer "F.Cu") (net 1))
 (segment (start 142.25 84.44) (end 142.54 84.73) (width 1) (layer "F.Cu") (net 1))
 (segment (start 133.14137 113.73) (end 116.54 113.73) (width 1) (layer "F.Cu") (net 1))
 (segment (start 172.04 84.73) (end 174.54 82.23) (width 1) (layer "F.Cu") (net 1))
 (segment (start 110 78.27) (end 110 84.69) (width 1) (layer "F.Cu") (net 1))
 (segment (start 103.54 84.73) (end 110.04 84.73) (width 1) (layer "F.Cu") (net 1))
 (segment (start 145.9275 113.8425) (end 146.04 113.73) (width 1) (layer "F.Cu") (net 1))
 (segment (start 166.66 112.11) (end 171.96 112.11) (width 1) (layer "F.Cu") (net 1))
 (segment (start 165.04 127.73) (end 168.47 131.16) (width 1) (layer "F.Cu") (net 1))
 (segment (start 145.9275 119.15) (end 145.9275 113.8425) (width 1) (layer "F.Cu") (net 1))
 (segment (start 101.33 93.61) (end 101.33 86.94) (width 1) (layer "F.Cu") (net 1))
 (segment (start 165.04 113.73) (end 166.66 112.11) (width 1) (layer "F.Cu") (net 1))
 (segment (start 166.66 97.11) (end 168.33 95.44) (width 1) (layer "F.Cu") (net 1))
 (segment (start 168.47 131.16) (end 171.96 131.16) (width 1) (layer "F.Cu") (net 1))
 (segment (start 136.89 108.85) (end 136.89 109.98137) (width 1) (layer "F.Cu") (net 1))
 (segment (start 115.08 115.27) (end 115.08 119.15) (width 1) (layer "F.Cu") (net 1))
 (segment (start 168.33 95.44) (end 176.515 95.44) (width 1) (layer "F.Cu") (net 1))
 (segment (start 142.54 84.73) (end 172.04 84.73) (width 1) (layer "F.Cu") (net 1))
 (segment (start 110 84.69) (end 110.04 84.73) (width 1) (layer "F.Cu") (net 1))
 (segment (start 133.14137 113.73) (end 146.04 113.73) (width 1) (layer "F.Cu") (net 1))
 (segment (start 142.25 78.27) (end 142.25 84.44) (width 1) (layer "F.Cu") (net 1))
 (segment (start 146.04 113.73) (end 165.04 113.73) (width 1) (layer "F.Cu") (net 1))
 (segment (start 101.33 86.94) (end 103.54 84.73) (width 1) (layer "F.Cu") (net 1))
 (segment (start 174.54 82.23) (end 174.54 81.23) (width 1) (layer "F.Cu") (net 1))
 (segment (start 116.54 113.73) (end 115.04 115.23) (width 1) (layer "F.Cu") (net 1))
 (segment (start 136.89 109.98137) (end 133.14137 113.73) (width 1) (layer "F.Cu") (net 1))
 (segment (start 174.54 81.23) (end 174.5 81.19) (width 1) (layer "F.Cu") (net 1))
 (segment (start 174.5 81.19) (end 174.5 78.27) (width 1) (layer "F.Cu") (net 1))
 (segment (start 161.04 88.73) (end 178.54 88.73) (width 1) (layer "B.Cu") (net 6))
 (segment (start 180.85 86.42) (end 178.54 88.73) (width 1) (layer "B.Cu") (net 6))
 (segment (start 159.75 90.02) (end 161.04 88.73) (width 1) (layer "B.Cu") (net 6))
 (segment (start 180.85 75.73) (end 180.85 86.42) (width 1) (layer "B.Cu") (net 6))
 (segment (start 159.75 93.61) (end 159.75 90.02) (width 1) (layer "B.Cu") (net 6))
 (segment (start 154.04 82.23) (end 150.04 82.23) (width 1) (layer "B.Cu") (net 7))
 (segment (start 157.21 93.61) (end 157.21 85.4) (width 1) (layer "B.Cu") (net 7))
 (segment (start 148.6 80.79) (end 148.6 75.73) (width 1) (layer "B.Cu") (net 7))
 (segment (start 157.21 85.4) (end 154.04 82.23) (width 1) (layer "B.Cu") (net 7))
 (segment (start 150.04 82.23) (end 148.6 80.79) (width 1) (layer "B.Cu") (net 7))
 (segment (start 116.35 86.04) (end 119.04 88.73) (width 1) (layer "B.Cu") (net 3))
 (segment (start 153.04 88.73) (end 154.67 90.36) (width 1) (layer "B.Cu") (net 3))
 (segment (start 154.67 90.36) (end 154.67 93.61) (width 1) (layer "B.Cu") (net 3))
 (segment (start 116.35 75.73) (end 116.35 86.04) (width 1) (layer "B.Cu") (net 3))
 (segment (start 119.04 88.73) (end 153.04 88.73) (width 1) (layer "B.Cu") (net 3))
 (segment (start 108.73 115.54) (end 111.04 113.23) (width 1) (layer "B.Cu") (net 5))
 (segment (start 140.04 111.73) (end 150.38137 111.73) (width 1) (layer "B.Cu") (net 5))
 (segment (start 152.13 109.98137) (end 152.13 108.85) (width 1) (layer "B.Cu") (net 5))
 (segment (start 108.73 121.69) (end 108.73 115.54) (width 1) (layer "B.Cu") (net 5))
 (segment (start 138.54 113.23) (end 140.04 111.73) (width 1) (layer "B.Cu") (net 5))
 (segment (start 150.38137 111.73) (end 152.13 109.98137) (width 1) (layer "B.Cu") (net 5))
 (segment (start 111.04 113.23) (end 138.54 113.23) (width 1) (layer "B.Cu") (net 5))
 (segment (start 152.04 114.23) (end 154.67 111.6) (width 1) (layer "B.Cu") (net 9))
 (segment (start 154.67 111.6) (end 154.67 108.85) (width 1) (layer "B.Cu") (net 9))
 (segment (start 139.5775 117.1925) (end 142.54 114.23) (width 1) (layer "B.Cu") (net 9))
 (segment (start 139.5775 121.69) (end 139.5775 117.1925) (width 1) (layer "B.Cu") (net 9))
 (segment (start 142.54 114.23) (end 152.04 114.23) (width 1) (layer "B.Cu") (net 9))
 (segment (start 163.27 118.46) (end 174.5 118.46) (width 1) (layer "B.Cu") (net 2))
 (segment (start 159.75 114.94) (end 163.27 118.46) (width 1) (layer "B.Cu") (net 2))
 (segment (start 159.75 108.85) (end 159.75 114.94) (width 1) (layer "B.Cu") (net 2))
 (segment (start 157.21 108.85) (end 157.21 128.4) (width 1) (layer "B.Cu") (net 8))
 (segment (start 157.21 128.4) (end 166.32 137.51) (width 1) (layer "B.Cu") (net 8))
 (segment (start 166.32 137.51) (end 174.5 137.51) (width 1) (layer "B.Cu") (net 8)))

